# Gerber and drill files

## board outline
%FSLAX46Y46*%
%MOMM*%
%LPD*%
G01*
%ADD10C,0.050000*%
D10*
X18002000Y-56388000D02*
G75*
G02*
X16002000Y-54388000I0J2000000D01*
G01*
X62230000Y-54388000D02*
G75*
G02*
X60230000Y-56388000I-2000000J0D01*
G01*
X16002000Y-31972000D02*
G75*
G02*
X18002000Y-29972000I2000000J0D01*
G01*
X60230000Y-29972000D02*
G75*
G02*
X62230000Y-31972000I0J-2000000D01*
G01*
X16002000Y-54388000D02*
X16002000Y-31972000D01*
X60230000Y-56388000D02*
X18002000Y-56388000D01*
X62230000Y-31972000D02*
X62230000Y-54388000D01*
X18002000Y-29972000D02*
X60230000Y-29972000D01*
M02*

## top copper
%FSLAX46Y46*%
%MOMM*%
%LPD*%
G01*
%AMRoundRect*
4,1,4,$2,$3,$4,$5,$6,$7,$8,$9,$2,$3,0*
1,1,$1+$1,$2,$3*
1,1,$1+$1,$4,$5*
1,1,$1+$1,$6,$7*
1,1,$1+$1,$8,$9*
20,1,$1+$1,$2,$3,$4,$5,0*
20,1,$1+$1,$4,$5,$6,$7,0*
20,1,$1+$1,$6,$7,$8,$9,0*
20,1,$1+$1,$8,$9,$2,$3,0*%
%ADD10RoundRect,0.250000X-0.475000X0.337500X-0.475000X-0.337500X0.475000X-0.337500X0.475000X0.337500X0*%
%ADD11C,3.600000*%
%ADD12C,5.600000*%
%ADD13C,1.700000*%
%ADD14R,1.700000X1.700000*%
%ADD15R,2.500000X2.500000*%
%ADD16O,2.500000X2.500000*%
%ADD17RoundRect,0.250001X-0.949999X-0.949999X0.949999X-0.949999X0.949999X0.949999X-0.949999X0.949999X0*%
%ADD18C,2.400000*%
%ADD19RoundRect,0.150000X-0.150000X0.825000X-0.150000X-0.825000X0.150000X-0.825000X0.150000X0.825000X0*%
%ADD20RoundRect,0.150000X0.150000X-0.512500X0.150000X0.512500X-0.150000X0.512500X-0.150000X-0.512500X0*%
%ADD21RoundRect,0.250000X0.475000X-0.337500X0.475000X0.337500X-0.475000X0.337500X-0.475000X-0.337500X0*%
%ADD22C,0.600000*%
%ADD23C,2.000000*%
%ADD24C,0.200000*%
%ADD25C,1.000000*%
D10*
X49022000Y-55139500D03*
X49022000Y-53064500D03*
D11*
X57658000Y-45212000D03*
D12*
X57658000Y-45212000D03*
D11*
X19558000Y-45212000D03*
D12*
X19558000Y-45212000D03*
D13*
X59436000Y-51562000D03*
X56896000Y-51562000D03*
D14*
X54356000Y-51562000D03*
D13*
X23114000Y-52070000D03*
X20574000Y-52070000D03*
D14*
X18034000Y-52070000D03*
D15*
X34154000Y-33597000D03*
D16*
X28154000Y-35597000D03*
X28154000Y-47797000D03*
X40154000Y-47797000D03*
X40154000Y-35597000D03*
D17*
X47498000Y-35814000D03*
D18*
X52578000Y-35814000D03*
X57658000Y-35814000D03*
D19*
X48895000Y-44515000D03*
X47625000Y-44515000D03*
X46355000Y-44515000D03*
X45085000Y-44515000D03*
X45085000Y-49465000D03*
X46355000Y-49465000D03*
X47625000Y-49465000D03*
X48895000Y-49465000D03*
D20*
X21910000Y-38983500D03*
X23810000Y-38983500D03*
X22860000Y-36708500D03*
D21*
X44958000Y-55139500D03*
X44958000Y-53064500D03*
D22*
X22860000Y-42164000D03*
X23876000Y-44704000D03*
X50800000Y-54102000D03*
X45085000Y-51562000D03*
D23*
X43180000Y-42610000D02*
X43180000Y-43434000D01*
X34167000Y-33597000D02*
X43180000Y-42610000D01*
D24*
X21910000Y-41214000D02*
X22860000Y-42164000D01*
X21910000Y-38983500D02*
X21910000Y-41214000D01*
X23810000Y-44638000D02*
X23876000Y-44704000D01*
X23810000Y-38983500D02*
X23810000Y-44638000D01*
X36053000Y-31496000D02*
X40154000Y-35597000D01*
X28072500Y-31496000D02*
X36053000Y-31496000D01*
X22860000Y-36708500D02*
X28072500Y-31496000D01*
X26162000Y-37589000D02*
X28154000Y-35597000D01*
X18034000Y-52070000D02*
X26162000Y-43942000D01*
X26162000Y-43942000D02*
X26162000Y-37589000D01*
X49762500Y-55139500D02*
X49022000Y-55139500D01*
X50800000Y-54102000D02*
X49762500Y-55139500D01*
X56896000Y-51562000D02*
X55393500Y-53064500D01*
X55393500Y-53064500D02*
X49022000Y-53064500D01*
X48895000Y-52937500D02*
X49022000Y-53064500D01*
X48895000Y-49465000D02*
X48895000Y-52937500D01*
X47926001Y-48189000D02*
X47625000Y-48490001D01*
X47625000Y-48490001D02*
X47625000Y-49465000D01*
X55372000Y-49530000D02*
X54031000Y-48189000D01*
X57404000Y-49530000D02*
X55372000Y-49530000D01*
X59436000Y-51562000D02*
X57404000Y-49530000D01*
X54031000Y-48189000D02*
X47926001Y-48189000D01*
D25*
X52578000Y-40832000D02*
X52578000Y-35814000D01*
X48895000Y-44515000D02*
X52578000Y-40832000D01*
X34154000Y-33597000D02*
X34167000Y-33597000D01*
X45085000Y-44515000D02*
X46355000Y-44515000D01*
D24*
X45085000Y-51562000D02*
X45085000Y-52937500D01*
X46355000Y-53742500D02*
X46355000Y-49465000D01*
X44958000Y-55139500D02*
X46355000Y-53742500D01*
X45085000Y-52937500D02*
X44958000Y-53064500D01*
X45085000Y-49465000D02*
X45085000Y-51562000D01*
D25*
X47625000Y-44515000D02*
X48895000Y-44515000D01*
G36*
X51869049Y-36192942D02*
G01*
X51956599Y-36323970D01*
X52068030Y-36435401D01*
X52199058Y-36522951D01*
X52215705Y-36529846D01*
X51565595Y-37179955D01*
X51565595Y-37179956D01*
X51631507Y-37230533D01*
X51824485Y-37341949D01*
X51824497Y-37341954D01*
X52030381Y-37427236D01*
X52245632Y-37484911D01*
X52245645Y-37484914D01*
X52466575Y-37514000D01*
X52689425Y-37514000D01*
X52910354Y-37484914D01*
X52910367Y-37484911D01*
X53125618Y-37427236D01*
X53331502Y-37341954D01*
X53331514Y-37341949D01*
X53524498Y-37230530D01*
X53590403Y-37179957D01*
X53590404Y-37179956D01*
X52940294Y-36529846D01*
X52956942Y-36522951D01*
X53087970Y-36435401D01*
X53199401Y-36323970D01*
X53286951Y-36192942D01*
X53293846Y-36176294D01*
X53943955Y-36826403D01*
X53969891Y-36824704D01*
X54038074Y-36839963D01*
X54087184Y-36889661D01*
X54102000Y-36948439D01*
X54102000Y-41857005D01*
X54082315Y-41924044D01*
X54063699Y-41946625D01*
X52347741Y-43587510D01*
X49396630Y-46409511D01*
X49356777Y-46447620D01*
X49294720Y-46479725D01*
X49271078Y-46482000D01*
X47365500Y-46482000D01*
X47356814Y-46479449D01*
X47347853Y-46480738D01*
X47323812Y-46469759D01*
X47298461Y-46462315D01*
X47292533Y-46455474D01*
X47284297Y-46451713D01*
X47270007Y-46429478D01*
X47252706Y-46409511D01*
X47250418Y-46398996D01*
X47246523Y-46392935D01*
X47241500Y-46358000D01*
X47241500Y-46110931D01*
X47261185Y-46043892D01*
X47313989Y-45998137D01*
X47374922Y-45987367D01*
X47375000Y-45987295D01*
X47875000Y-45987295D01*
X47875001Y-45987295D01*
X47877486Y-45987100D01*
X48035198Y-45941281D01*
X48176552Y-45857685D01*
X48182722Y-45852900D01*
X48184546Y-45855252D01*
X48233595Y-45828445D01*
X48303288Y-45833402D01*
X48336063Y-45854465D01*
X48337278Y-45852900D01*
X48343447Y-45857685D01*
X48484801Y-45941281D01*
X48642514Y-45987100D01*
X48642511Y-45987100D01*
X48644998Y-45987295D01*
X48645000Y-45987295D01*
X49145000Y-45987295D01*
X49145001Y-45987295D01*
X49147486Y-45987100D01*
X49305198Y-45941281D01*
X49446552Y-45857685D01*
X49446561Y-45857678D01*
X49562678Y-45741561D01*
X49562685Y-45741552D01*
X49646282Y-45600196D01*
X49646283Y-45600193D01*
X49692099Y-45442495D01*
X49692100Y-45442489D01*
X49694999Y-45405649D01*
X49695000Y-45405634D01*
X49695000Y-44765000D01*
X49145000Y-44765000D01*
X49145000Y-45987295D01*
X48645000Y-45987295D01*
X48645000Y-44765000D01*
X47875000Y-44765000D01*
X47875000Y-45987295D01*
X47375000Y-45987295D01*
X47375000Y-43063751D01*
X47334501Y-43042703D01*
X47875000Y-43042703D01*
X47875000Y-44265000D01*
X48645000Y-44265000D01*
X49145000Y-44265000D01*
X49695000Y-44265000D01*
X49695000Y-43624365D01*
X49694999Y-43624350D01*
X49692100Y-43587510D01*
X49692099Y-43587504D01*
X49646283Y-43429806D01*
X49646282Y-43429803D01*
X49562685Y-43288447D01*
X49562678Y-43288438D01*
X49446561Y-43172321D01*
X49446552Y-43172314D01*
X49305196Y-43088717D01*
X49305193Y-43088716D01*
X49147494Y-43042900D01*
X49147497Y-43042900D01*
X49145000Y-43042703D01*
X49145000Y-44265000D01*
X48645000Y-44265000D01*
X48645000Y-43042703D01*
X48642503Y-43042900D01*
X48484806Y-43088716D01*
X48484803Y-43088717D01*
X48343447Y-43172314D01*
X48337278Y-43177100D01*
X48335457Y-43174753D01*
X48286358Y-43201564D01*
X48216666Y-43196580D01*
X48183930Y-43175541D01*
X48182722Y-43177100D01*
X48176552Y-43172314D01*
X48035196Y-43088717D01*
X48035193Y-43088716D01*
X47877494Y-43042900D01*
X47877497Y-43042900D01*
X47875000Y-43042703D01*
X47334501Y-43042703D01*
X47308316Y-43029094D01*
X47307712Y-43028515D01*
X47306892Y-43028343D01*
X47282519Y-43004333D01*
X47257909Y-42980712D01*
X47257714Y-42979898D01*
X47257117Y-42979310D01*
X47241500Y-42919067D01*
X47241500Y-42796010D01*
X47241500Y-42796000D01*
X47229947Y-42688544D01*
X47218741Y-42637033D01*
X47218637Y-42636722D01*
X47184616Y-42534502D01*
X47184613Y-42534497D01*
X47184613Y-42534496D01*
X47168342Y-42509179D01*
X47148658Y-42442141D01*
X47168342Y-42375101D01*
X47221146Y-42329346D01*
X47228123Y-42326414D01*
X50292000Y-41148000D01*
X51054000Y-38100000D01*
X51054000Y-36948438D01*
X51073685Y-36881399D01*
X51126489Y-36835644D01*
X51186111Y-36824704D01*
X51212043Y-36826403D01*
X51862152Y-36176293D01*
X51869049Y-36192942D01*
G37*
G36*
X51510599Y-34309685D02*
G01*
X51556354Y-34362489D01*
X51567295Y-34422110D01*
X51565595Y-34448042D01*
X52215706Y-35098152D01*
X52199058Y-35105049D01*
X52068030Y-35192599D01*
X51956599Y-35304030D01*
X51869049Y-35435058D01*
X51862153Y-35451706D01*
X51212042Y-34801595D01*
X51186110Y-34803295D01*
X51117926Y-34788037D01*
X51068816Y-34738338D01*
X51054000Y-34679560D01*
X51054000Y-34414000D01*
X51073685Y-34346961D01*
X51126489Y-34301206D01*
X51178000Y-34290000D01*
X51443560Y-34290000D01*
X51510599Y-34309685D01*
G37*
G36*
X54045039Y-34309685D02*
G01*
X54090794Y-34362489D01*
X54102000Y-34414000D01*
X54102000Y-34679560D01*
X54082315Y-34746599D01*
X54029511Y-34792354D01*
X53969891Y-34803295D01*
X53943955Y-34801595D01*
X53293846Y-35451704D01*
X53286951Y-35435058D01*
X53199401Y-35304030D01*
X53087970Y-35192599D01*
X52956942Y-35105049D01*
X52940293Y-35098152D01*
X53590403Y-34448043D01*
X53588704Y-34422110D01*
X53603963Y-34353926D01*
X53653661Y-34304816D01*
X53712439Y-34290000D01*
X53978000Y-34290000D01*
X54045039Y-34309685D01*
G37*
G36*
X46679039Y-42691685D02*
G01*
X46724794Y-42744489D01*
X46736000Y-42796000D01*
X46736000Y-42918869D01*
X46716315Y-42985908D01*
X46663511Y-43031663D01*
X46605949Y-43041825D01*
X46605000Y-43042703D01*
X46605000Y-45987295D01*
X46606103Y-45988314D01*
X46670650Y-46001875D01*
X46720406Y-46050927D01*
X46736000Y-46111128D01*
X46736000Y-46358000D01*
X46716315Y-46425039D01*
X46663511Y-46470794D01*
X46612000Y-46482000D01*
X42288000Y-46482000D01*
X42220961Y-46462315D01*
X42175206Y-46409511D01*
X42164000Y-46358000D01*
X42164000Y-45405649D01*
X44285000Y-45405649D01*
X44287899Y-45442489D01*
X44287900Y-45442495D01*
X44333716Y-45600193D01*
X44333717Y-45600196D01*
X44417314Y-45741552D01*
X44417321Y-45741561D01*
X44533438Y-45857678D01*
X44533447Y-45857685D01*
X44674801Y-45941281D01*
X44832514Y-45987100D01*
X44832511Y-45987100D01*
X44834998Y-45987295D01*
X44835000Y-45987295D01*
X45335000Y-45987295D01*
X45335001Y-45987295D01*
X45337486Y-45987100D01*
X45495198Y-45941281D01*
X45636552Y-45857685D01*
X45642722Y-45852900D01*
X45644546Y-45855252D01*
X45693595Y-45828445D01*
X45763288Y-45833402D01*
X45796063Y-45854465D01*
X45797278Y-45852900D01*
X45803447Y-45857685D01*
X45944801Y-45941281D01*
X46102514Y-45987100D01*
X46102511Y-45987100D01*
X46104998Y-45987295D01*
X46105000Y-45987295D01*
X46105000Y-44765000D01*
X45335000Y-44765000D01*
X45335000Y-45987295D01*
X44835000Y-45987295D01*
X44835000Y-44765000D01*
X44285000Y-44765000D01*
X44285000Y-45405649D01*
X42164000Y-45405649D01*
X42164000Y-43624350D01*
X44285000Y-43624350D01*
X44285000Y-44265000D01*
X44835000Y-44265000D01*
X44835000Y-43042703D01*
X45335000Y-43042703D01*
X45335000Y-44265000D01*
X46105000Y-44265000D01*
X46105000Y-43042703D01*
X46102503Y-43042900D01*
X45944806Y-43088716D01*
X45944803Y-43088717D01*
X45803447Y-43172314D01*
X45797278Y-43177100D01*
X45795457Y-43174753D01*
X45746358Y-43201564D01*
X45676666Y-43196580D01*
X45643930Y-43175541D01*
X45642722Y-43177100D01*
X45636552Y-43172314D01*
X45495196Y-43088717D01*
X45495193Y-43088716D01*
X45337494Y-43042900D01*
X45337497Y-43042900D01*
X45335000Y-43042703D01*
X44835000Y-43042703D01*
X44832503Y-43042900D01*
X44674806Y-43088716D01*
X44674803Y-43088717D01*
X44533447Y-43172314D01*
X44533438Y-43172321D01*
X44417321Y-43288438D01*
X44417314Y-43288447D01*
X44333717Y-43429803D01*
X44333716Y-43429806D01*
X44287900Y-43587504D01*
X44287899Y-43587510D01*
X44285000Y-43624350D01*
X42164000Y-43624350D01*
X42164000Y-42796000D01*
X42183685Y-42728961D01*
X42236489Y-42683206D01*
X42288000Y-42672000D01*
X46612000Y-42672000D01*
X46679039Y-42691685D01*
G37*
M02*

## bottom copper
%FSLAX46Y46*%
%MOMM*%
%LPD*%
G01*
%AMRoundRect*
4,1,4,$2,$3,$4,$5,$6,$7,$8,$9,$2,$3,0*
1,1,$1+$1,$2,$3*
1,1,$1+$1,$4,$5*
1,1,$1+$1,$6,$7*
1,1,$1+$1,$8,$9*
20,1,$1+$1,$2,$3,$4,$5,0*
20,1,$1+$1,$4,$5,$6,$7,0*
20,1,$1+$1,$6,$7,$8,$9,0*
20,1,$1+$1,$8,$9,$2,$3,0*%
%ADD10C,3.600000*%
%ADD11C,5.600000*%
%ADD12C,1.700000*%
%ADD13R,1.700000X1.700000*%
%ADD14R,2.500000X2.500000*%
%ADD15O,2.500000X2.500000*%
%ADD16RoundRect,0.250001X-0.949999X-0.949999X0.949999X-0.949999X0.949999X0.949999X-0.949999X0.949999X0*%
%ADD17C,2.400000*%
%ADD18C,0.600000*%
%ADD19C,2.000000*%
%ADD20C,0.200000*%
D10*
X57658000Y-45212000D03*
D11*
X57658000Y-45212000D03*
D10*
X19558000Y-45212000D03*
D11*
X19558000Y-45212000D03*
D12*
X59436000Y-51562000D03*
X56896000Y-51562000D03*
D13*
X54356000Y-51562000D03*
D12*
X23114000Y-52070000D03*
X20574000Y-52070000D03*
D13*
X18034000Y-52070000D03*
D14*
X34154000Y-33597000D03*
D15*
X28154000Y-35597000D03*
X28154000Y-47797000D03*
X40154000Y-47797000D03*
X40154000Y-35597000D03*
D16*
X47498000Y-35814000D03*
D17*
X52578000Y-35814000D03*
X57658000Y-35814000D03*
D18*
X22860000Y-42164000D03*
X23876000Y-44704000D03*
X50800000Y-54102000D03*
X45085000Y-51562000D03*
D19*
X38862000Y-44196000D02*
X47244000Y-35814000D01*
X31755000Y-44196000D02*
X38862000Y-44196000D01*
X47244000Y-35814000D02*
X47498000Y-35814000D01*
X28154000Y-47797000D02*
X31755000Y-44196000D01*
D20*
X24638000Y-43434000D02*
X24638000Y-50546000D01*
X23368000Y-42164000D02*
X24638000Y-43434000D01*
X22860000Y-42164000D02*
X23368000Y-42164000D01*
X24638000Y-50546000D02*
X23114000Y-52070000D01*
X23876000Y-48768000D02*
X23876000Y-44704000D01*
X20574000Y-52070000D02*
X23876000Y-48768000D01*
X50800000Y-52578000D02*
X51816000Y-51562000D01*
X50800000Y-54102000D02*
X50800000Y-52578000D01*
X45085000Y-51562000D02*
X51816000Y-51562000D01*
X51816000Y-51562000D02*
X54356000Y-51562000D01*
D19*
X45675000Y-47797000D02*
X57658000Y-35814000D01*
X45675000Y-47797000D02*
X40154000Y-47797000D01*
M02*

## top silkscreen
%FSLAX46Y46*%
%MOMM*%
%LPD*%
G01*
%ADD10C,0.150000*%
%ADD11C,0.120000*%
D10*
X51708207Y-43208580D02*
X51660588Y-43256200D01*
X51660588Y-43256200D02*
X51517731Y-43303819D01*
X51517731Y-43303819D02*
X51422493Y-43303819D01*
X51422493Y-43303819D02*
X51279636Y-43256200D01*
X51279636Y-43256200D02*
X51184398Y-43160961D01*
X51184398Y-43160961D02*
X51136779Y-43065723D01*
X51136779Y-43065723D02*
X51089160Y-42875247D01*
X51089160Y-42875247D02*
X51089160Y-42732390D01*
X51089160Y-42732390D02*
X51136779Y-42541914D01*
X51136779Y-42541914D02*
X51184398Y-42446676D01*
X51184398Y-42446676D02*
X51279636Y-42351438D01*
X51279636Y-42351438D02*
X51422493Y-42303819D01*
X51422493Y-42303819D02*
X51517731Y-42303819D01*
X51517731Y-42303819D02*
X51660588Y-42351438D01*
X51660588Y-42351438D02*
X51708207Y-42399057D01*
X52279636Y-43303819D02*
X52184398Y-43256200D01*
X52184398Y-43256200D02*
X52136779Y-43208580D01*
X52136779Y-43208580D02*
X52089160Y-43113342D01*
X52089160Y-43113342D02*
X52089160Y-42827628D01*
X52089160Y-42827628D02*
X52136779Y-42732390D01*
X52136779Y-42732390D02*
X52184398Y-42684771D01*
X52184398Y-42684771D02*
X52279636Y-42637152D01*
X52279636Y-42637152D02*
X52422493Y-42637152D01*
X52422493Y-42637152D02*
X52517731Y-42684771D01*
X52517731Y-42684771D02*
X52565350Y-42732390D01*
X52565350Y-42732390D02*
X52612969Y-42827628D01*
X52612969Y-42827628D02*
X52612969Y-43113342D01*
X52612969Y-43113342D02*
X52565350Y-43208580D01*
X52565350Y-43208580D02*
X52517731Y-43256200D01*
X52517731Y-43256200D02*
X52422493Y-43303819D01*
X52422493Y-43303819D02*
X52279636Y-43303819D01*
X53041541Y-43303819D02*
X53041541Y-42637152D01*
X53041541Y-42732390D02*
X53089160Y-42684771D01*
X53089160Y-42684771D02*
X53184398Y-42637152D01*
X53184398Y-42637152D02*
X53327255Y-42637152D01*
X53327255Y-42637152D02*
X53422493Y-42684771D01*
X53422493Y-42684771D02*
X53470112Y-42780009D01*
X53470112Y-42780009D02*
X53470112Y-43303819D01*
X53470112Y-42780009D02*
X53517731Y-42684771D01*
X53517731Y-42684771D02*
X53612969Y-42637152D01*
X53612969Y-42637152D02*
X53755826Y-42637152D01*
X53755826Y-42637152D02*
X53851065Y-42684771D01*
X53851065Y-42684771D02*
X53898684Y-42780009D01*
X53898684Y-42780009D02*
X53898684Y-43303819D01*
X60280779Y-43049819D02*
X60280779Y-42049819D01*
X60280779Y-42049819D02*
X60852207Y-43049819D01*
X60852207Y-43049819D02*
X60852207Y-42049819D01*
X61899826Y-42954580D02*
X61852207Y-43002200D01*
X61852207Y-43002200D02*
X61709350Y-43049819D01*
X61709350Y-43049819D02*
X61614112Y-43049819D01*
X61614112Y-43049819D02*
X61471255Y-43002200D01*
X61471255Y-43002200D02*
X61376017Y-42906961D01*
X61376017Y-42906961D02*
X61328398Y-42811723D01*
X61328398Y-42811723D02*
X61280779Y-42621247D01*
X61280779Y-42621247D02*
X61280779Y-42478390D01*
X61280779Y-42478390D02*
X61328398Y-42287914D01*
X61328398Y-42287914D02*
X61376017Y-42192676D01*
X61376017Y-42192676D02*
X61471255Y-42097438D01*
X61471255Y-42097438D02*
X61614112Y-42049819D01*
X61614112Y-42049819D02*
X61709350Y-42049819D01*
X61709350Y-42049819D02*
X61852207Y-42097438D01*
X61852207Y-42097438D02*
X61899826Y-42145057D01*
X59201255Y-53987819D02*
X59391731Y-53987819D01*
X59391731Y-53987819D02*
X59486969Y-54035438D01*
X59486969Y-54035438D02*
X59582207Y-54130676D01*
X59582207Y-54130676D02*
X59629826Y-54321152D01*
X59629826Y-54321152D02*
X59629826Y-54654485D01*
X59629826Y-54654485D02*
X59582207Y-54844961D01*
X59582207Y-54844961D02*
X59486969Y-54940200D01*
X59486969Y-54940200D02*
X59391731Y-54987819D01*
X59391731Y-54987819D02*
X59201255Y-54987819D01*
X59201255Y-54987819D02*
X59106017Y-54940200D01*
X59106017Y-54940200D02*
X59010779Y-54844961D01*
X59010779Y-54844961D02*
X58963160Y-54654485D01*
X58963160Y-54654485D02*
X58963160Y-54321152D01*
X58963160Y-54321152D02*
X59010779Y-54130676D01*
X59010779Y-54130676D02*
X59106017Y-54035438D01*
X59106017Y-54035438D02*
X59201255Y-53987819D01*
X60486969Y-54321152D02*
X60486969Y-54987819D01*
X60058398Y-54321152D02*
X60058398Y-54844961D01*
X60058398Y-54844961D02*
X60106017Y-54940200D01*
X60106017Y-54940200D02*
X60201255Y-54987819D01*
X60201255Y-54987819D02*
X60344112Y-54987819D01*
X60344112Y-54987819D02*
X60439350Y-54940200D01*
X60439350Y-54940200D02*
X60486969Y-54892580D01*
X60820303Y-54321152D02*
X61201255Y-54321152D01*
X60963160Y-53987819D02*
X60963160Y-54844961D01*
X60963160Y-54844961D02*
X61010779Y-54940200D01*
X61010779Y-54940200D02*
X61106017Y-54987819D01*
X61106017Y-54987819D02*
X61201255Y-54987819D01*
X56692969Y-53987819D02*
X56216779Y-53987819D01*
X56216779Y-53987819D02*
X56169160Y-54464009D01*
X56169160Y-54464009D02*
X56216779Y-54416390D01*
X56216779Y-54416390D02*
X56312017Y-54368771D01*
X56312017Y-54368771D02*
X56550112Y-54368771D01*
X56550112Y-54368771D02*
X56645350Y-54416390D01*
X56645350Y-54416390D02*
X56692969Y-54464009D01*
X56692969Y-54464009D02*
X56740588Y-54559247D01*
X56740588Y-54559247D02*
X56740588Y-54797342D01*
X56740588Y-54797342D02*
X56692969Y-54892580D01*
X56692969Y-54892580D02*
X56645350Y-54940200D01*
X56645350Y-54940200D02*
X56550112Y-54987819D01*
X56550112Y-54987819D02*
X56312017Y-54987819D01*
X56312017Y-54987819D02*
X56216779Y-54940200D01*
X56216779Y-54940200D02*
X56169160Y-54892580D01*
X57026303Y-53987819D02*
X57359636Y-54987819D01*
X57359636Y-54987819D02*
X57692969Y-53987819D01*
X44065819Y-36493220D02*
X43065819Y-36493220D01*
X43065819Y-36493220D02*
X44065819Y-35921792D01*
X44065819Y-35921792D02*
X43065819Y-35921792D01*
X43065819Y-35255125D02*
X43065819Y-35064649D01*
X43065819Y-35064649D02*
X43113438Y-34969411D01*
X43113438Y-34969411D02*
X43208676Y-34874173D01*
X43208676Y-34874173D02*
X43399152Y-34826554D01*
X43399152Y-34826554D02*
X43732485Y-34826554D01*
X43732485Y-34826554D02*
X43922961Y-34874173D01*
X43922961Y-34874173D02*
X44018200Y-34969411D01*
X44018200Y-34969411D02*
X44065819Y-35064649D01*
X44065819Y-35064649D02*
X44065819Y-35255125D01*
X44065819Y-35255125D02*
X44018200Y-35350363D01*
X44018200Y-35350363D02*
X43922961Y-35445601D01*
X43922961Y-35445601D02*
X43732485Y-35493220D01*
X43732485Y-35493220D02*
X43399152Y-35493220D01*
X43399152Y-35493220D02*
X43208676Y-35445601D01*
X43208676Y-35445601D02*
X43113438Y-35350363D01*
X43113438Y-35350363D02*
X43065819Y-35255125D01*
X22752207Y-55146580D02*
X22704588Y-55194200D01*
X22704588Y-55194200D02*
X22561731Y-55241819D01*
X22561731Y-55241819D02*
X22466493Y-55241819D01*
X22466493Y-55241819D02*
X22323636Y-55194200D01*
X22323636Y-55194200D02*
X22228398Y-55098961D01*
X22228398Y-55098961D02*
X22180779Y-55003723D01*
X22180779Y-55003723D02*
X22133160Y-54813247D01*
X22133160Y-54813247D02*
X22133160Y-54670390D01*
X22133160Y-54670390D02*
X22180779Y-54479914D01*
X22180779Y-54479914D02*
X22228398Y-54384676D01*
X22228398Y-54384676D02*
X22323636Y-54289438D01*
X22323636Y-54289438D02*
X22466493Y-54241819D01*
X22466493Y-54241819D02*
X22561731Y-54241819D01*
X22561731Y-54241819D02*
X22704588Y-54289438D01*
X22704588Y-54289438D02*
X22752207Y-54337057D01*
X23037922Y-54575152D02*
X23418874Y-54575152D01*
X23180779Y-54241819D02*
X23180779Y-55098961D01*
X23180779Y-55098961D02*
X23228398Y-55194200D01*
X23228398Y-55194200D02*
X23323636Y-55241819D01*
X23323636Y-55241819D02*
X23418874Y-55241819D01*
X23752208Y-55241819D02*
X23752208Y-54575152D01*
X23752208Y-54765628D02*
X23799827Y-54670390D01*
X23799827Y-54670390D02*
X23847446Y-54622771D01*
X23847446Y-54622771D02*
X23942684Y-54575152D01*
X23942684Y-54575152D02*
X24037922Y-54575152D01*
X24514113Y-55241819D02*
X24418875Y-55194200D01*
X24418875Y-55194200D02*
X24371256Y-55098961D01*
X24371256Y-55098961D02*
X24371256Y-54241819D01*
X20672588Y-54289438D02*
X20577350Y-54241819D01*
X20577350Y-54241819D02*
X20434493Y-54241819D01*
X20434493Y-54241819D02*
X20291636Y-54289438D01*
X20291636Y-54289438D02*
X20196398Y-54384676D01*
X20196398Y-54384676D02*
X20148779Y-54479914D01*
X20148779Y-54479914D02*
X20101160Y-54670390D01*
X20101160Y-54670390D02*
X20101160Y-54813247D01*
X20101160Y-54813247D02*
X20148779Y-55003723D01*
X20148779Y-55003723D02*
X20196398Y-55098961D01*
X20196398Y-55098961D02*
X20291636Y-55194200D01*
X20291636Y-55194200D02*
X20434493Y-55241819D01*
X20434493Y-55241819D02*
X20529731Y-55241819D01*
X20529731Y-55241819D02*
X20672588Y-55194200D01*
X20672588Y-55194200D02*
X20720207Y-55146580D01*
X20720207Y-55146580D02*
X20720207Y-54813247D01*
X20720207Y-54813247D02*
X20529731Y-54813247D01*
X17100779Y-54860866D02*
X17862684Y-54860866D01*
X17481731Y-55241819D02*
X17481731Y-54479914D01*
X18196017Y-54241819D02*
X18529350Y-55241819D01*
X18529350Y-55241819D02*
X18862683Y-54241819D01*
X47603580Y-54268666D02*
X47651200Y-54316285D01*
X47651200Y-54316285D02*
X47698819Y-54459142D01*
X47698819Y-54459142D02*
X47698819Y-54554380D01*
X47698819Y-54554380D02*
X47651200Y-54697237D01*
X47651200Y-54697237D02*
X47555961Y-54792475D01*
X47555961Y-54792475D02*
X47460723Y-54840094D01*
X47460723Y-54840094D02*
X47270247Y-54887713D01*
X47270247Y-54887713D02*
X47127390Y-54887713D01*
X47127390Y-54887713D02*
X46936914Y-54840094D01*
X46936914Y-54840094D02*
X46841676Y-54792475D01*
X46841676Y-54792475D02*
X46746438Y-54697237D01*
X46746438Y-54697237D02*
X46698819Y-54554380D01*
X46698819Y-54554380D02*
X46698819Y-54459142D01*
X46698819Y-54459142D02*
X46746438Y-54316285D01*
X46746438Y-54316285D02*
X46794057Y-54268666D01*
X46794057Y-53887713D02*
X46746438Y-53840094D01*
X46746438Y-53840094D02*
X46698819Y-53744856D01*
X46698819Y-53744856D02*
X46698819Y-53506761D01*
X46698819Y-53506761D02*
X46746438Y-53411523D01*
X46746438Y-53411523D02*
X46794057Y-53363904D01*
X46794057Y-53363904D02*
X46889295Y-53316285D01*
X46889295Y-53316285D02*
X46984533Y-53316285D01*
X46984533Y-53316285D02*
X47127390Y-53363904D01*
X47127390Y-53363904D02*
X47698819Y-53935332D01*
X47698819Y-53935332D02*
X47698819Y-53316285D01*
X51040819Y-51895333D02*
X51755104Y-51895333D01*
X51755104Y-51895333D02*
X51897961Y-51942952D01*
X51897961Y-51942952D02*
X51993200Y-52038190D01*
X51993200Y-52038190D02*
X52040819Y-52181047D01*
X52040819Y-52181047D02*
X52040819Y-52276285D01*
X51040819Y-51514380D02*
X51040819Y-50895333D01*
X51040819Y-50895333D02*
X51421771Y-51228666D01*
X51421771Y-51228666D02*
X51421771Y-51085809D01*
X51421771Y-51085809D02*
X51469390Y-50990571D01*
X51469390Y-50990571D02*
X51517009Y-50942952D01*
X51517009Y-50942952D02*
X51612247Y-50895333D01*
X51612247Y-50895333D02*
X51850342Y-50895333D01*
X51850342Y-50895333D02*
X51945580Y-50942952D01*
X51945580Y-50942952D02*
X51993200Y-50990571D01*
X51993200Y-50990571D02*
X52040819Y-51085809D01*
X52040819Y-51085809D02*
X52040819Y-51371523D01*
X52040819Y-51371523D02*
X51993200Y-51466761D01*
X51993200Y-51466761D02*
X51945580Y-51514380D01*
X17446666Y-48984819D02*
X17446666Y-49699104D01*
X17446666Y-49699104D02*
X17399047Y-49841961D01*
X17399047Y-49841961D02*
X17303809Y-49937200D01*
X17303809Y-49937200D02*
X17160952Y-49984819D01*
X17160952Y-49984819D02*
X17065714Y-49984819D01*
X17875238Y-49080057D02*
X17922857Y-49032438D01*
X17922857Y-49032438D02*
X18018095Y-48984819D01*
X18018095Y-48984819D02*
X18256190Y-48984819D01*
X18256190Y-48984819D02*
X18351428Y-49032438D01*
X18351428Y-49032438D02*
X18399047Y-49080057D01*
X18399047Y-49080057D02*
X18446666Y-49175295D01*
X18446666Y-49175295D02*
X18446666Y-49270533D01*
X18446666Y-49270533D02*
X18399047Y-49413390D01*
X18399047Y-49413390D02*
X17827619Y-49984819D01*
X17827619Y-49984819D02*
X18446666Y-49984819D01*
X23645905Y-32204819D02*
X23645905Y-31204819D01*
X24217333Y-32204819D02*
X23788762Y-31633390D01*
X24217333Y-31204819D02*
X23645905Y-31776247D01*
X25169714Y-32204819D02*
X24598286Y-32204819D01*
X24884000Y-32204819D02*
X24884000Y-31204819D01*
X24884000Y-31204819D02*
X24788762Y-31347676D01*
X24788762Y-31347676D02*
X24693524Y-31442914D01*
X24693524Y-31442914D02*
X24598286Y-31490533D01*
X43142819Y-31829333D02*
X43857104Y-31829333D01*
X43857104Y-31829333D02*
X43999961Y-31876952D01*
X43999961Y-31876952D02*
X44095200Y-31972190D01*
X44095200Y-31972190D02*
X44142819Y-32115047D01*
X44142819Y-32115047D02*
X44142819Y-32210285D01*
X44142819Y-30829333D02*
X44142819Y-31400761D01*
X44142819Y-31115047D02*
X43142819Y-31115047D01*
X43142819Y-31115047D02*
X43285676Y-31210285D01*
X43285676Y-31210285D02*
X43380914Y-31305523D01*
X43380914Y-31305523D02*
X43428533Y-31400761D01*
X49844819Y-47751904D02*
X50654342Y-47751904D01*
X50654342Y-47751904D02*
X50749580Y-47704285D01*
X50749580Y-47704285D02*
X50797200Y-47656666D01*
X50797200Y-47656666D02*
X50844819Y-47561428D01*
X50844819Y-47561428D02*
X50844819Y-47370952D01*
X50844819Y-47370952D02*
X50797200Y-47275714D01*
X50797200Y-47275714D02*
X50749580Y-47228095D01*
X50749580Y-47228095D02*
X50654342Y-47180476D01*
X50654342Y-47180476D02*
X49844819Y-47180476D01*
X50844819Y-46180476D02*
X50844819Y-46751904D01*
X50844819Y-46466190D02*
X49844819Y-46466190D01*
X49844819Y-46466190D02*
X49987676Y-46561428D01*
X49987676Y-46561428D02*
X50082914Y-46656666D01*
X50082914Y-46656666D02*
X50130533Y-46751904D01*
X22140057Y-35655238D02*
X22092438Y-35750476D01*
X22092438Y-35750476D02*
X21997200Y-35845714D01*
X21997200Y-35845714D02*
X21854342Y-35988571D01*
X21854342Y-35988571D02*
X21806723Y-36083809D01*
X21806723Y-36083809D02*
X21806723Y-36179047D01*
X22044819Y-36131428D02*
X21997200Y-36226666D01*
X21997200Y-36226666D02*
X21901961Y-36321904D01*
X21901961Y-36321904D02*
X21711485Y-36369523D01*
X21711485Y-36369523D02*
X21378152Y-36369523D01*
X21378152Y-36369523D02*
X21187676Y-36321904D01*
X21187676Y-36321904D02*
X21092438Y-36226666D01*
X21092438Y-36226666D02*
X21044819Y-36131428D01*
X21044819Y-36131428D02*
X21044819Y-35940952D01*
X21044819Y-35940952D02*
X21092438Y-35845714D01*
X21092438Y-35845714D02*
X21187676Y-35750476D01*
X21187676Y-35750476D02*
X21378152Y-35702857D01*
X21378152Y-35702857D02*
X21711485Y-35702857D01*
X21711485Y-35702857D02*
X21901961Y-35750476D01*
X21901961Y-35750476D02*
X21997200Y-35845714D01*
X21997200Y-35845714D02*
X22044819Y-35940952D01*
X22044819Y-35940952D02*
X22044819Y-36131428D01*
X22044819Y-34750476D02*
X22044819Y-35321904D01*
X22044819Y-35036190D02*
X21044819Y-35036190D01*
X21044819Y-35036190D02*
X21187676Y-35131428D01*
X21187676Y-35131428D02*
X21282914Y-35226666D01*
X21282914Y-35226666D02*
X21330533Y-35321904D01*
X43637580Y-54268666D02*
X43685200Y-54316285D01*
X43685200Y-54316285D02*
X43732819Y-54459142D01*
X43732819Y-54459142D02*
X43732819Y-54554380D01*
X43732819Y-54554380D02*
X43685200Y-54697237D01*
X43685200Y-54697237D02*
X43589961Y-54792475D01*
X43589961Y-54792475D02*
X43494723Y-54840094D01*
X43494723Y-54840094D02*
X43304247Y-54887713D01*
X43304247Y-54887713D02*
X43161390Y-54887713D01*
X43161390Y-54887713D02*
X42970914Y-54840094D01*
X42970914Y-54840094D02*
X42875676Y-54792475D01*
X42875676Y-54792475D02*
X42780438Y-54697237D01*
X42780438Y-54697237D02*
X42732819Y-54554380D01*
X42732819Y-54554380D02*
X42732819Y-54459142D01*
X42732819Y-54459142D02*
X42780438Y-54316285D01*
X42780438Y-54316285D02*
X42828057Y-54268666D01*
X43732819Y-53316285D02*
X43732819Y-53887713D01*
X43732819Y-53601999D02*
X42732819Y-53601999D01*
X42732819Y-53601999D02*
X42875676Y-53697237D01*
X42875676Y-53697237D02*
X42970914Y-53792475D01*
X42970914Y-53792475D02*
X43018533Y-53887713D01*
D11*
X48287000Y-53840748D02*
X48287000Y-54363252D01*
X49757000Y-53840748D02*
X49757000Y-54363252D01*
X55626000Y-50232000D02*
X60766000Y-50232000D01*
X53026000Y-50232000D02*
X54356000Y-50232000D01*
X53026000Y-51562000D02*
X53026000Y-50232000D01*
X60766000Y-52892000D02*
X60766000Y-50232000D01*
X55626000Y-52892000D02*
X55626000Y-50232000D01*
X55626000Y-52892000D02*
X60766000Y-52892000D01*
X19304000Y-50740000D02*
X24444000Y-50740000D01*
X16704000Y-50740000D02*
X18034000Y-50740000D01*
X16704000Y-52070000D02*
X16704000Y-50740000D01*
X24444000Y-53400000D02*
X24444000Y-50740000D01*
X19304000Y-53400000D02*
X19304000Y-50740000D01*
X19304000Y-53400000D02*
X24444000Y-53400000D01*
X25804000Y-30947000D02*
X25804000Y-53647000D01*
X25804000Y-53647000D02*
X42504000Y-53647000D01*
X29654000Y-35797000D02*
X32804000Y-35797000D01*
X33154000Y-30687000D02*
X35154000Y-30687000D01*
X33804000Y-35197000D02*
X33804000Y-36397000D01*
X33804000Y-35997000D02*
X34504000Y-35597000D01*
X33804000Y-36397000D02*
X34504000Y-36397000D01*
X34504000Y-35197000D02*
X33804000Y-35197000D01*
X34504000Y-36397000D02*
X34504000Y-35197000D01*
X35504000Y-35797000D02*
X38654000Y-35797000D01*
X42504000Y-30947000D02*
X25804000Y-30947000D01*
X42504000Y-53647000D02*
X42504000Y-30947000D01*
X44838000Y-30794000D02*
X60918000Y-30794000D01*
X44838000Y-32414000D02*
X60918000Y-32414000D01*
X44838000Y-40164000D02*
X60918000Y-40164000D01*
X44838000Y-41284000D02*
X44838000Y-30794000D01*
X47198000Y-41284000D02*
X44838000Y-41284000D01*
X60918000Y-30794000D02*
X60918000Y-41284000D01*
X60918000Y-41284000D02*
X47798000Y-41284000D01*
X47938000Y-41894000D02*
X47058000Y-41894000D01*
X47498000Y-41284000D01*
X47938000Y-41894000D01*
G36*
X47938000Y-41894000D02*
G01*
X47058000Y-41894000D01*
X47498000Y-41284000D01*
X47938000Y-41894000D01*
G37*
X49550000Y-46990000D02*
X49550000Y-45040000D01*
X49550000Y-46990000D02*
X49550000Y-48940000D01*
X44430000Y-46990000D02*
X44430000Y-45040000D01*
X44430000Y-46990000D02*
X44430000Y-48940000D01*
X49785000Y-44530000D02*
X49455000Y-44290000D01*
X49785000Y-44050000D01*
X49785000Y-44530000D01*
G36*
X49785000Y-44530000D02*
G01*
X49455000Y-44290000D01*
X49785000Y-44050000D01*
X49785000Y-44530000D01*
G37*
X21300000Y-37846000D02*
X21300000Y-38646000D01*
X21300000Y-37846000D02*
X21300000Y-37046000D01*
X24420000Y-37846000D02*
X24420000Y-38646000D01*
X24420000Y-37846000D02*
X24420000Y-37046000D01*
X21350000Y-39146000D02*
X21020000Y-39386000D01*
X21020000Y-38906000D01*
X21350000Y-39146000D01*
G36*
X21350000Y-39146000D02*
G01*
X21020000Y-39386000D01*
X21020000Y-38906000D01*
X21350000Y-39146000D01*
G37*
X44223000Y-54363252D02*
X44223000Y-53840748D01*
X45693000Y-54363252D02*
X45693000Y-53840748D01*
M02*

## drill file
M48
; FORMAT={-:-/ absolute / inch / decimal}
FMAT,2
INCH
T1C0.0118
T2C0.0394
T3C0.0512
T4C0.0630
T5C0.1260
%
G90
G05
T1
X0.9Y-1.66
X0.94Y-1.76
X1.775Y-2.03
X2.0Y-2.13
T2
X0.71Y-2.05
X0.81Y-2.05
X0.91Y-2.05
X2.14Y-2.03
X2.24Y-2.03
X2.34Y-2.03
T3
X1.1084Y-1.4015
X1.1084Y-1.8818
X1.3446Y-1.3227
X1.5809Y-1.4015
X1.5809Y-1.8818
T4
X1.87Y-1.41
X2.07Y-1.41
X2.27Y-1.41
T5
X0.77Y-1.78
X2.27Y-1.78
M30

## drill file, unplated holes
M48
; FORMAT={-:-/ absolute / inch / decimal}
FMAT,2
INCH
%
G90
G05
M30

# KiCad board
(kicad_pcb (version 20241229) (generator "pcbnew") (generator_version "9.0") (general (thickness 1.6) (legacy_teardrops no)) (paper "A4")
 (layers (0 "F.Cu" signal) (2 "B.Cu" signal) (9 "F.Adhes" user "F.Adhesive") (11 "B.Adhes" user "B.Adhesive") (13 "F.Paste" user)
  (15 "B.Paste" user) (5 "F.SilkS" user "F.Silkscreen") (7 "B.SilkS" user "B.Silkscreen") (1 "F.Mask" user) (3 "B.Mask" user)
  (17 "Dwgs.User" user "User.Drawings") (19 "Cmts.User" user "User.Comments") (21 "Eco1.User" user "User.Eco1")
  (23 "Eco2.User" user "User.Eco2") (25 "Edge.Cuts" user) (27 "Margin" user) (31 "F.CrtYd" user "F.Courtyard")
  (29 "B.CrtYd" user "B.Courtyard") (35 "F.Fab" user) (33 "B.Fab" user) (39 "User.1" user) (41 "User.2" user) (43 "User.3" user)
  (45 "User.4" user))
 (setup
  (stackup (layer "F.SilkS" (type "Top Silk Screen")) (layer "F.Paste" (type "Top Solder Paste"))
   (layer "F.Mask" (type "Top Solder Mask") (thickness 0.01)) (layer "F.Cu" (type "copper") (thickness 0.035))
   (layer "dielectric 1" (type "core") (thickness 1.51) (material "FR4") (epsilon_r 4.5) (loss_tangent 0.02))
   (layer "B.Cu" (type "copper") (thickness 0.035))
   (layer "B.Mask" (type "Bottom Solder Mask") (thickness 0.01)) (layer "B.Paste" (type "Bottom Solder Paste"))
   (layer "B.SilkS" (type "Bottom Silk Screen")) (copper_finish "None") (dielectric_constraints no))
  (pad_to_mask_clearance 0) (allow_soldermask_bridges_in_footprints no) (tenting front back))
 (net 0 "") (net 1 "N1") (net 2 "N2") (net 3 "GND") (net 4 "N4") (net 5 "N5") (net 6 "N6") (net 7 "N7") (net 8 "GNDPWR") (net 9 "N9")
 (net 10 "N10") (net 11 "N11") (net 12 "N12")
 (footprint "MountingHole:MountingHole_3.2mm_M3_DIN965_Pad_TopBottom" (layer "F.Cu") (at 19.558 45.212)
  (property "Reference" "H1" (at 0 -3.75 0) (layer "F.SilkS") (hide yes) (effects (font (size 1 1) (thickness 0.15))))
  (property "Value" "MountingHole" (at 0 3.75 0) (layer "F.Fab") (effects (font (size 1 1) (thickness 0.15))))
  (pad "1" thru_hole circle (at 0 0) (size 3.6 3.6) (drill 3.2) (layers "*.Cu" "*.Mask") (remove_unused_layers no) (zone_connect 2))
  (pad "1" connect circle (at 0 0) (size 5.6 5.6) (layers "F.Cu" "F.Mask") (zone_connect 2))
  (pad "1" connect circle (at 0 0) (size 5.6 5.6) (layers "B.Cu" "B.Mask") (zone_connect 2)))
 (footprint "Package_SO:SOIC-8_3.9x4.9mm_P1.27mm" (layer "F.Cu") (at 46.99 46.99 -90)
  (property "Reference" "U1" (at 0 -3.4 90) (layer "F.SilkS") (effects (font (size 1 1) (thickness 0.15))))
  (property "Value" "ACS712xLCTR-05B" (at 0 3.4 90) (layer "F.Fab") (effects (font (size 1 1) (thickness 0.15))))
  (fp_line (start 0 2.56) (end -1.95 2.56) (stroke (width 0.12) (type solid)) (layer "F.SilkS"))
  (fp_line (start 0 2.56) (end 1.95 2.56) (stroke (width 0.12) (type solid)) (layer "F.SilkS"))
  (fp_line (start 0 -2.56) (end -1.95 -2.56) (stroke (width 0.12) (type solid)) (layer "F.SilkS"))
  (fp_line (start 0 -2.56) (end 1.95 -2.56) (stroke (width 0.12) (type solid)) (layer "F.SilkS"))
  (fp_poly (pts (xy -2.7 -2.465) (xy -2.94 -2.795) (xy -2.46 -2.795)) (stroke (width 0.12) (type solid)) (fill yes) (layer "F.SilkS"))
  (pad "1" smd roundrect (at -2.475 -1.905 270) (size 1.95 0.6) (layers "F.Cu" "F.Mask" "F.Paste") (roundrect_rratio 0.25) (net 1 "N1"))
  (pad "2" smd roundrect (at -2.475 -0.635 270) (size 1.95 0.6) (layers "F.Cu" "F.Mask" "F.Paste") (roundrect_rratio 0.25) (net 1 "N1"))
  (pad "3" smd roundrect (at -2.475 0.635 270) (size 1.95 0.6) (layers "F.Cu" "F.Mask" "F.Paste") (roundrect_rratio 0.25) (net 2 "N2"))
  (pad "4" smd roundrect (at -2.475 1.905 270) (size 1.95 0.6) (layers "F.Cu" "F.Mask" "F.Paste") (roundrect_rratio 0.25) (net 2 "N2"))
  (pad "5" smd roundrect (at 2.475 1.905 270) (size 1.95 0.6) (layers "F.Cu" "F.Mask" "F.Paste") (roundrect_rratio 0.25) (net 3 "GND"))
  (pad "6" smd roundrect (at 2.475 0.635 270) (size 1.95 0.6) (layers "F.Cu" "F.Mask" "F.Paste") (roundrect_rratio 0.25) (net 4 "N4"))
  (pad "7" smd roundrect (at 2.475 -0.635 270) (size 1.95 0.6) (layers "F.Cu" "F.Mask" "F.Paste") (roundrect_rratio 0.25) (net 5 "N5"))
  (pad "8" smd roundrect (at 2.475 -1.905 270) (size 1.95 0.6) (layers "F.Cu" "F.Mask" "F.Paste") (roundrect_rratio 0.25) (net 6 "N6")))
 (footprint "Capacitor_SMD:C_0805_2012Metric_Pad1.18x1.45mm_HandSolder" (layer "F.Cu") (at 44.958 54.102 90)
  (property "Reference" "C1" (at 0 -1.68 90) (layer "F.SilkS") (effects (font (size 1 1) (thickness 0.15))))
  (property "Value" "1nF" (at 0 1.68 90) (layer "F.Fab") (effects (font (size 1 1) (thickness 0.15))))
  (fp_line (start -0.261252 -0.735) (end 0.261252 -0.735) (stroke (width 0.12) (type solid)) (layer "F.SilkS"))
  (fp_line (start -0.261252 0.735) (end 0.261252 0.735) (stroke (width 0.12) (type solid)) (layer "F.SilkS"))
  (pad "1" smd roundrect (at -1.0375 0 90) (size 1.175 1.45) (layers "F.Cu" "F.Mask" "F.Paste") (roundrect_rratio 0.212766) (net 4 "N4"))
  (pad "2" smd roundrect (at 1.0375 0 90) (size 1.175 1.45) (layers "F.Cu" "F.Mask" "F.Paste") (roundrect_rratio 0.212766) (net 3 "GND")))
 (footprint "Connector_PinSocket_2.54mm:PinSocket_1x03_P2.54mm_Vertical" (layer "F.Cu") (at 18.034 52.07 90)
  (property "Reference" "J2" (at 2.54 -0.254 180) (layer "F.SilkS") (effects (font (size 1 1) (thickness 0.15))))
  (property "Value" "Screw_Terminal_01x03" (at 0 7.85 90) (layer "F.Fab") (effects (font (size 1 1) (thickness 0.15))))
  (fp_line (start 1.33 -1.33) (end 1.33 0) (stroke (width 0.12) (type solid)) (layer "F.SilkS"))
  (fp_line (start 0 -1.33) (end 1.33 -1.33) (stroke (width 0.12) (type solid)) (layer "F.SilkS"))
  (fp_line (start 1.33 1.27) (end 1.33 6.41) (stroke (width 0.12) (type solid)) (layer "F.SilkS"))
  (fp_line (start -1.33 1.27) (end 1.33 1.27) (stroke (width 0.12) (type solid)) (layer "F.SilkS"))
  (fp_line (start -1.33 1.27) (end -1.33 6.41) (stroke (width 0.12) (type solid)) (layer "F.SilkS"))
  (fp_line (start -1.33 6.41) (end 1.33 6.41) (stroke (width 0.12) (type solid)) (layer "F.SilkS"))
  (pad "1" thru_hole rect (at 0 0 90) (size 1.7 1.7) (drill 1) (layers "*.Cu" "*.Mask") (remove_unused_layers no) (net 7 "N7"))
  (pad "2" thru_hole circle (at 0 2.54 90) (size 1.7 1.7) (drill 1) (layers "*.Cu" "*.Mask") (remove_unused_layers no) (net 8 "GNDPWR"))
  (pad "3" thru_hole circle (at 0 5.08 90) (size 1.7 1.7) (drill 1) (layers "*.Cu" "*.Mask") (remove_unused_layers no) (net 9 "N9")))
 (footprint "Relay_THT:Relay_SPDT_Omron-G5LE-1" (layer "F.Cu") (at 34.154 33.597)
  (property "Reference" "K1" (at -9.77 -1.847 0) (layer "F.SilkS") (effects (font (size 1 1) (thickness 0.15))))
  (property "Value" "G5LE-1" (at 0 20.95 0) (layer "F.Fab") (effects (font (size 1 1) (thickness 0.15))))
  (fp_line (start -8.35 -2.65) (end -8.35 20.05) (stroke (width 0.12) (type solid)) (layer "F.SilkS"))
  (fp_line (start -8.35 20.05) (end 8.35 20.05) (stroke (width 0.12) (type solid)) (layer "F.SilkS"))
  (fp_line (start -4.5 2.2) (end -1.35 2.2) (stroke (width 0.12) (type solid)) (layer "F.SilkS"))
  (fp_line (start -1 -2.91) (end 1 -2.91) (stroke (width 0.12) (type solid)) (layer "F.SilkS"))
  (fp_line (start -0.35 1.6) (end -0.35 2.8) (stroke (width 0.12) (type solid)) (layer "F.SilkS"))
  (fp_line (start -0.35 2.4) (end 0.35 2) (stroke (width 0.12) (type solid)) (layer "F.SilkS"))
  (fp_line (start -0.35 2.8) (end 0.35 2.8) (stroke (width 0.12) (type solid)) (layer "F.SilkS"))
  (fp_line (start 0.35 1.6) (end -0.35 1.6) (stroke (width 0.12) (type solid)) (layer "F.SilkS"))
  (fp_line (start 0.35 2.8) (end 0.35 1.6) (stroke (width 0.12) (type solid)) (layer "F.SilkS"))
  (fp_line (start 1.35 2.2) (end 4.5 2.2) (stroke (width 0.12) (type solid)) (layer "F.SilkS"))
  (fp_line (start 8.35 -2.65) (end -8.35 -2.65) (stroke (width 0.12) (type solid)) (layer "F.SilkS"))
  (fp_line (start 8.35 20.05) (end 8.35 -2.65) (stroke (width 0.12) (type solid)) (layer "F.SilkS"))
  (pad "1" thru_hole rect (at 0 0) (size 2.5 2.5) (drill 1.3) (layers "*.Cu" "*.Mask") (remove_unused_layers no) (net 2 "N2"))
  (pad "2" thru_hole oval (at -6 2) (size 2.5 2.5) (drill 1.3) (layers "*.Cu" "*.Mask") (remove_unused_layers no) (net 7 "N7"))
  (pad "3" thru_hole oval (at -6 14.2) (size 2.5 2.5) (drill 1.3) (layers "*.Cu" "*.Mask") (remove_unused_layers no) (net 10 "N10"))
  (pad "4" thru_hole oval (at 6 14.2) (size 2.5 2.5) (drill 1.3) (layers "*.Cu" "*.Mask") (remove_unused_layers no) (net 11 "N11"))
  (pad "5" thru_hole oval (at 6 2) (size 2.5 2.5) (drill 1.3) (layers "*.Cu" "*.Mask") (remove_unused_layers no) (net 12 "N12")))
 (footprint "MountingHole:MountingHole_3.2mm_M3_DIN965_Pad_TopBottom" (layer "F.Cu") (at 57.658 45.212)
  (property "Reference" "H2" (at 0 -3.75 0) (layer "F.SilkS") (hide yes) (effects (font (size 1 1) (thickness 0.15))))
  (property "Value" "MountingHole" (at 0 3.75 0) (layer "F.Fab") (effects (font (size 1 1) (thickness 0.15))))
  (pad "1" thru_hole circle (at 0 0) (size 3.6 3.6) (drill 3.2) (layers "*.Cu" "*.Mask") (remove_unused_layers no) (zone_connect 2))
  (pad "1" connect circle (at 0 0) (size 5.6 5.6) (layers "F.Cu" "F.Mask") (zone_connect 2))
  (pad "1" connect circle (at 0 0) (size 5.6 5.6) (layers "B.Cu" "B.Mask") (zone_connect 2)))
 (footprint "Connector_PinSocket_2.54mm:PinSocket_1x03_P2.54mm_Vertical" (layer "F.Cu") (at 54.356 51.562 90)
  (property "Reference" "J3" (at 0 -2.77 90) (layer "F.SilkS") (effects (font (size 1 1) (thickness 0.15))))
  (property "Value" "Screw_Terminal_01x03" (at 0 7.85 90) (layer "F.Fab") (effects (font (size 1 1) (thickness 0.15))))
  (fp_line (start 1.33 -1.33) (end 1.33 0) (stroke (width 0.12) (type solid)) (layer "F.SilkS"))
  (fp_line (start 0 -1.33) (end 1.33 -1.33) (stroke (width 0.12) (type solid)) (layer "F.SilkS"))
  (fp_line (start 1.33 1.27) (end 1.33 6.41) (stroke (width 0.12) (type solid)) (layer "F.SilkS"))
  (fp_line (start -1.33 1.27) (end 1.33 1.27) (stroke (width 0.12) (type solid)) (layer "F.SilkS"))
  (fp_line (start -1.33 1.27) (end -1.33 6.41) (stroke (width 0.12) (type solid)) (layer "F.SilkS"))
  (fp_line (start -1.33 6.41) (end 1.33 6.41) (stroke (width 0.12) (type solid)) (layer "F.SilkS"))
  (pad "1" thru_hole rect (at 0 0 90) (size 1.7 1.7) (drill 1) (layers "*.Cu" "*.Mask") (remove_unused_layers no) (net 3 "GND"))
  (pad "2" thru_hole circle (at 0 2.54 90) (size 1.7 1.7) (drill 1) (layers "*.Cu" "*.Mask") (remove_unused_layers no) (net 6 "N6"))
  (pad "3" thru_hole circle (at 0 5.08 90) (size 1.7 1.7) (drill 1) (layers "*.Cu" "*.Mask") (remove_unused_layers no) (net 5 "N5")))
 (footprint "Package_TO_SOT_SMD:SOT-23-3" (layer "F.Cu") (at 22.86 37.846 90)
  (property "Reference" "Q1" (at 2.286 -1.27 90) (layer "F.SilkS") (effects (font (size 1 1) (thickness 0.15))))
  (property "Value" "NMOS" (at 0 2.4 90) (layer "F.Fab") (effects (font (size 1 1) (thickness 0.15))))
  (fp_line (start 0 -1.56) (end 0.8 -1.56) (stroke (width 0.12) (type solid)) (layer "F.SilkS"))
  (fp_line (start 0 -1.56) (end -0.8 -1.56) (stroke (width 0.12) (type solid)) (layer "F.SilkS"))
  (fp_line (start 0 1.56) (end 0.8 1.56) (stroke (width 0.12) (type solid)) (layer "F.SilkS"))
  (fp_line (start 0 1.56) (end -0.8 1.56) (stroke (width 0.12) (type solid)) (layer "F.SilkS"))
  (fp_poly (pts (xy -1.3 -1.51) (xy -1.54 -1.84) (xy -1.06 -1.84)) (stroke (width 0.12) (type solid)) (fill yes) (layer "F.SilkS"))
  (pad "1" smd roundrect (at -1.1375 -0.95 90) (size 1.325 0.6) (layers "F.Cu" "F.Mask" "F.Paste") (roundrect_rratio 0.25) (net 9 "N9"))
  (pad "2" smd roundrect (at -1.1375 0.95 90) (size 1.325 0.6) (layers "F.Cu" "F.Mask" "F.Paste") (roundrect_rratio 0.25) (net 8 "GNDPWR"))
  (pad "3" smd roundrect (at 1.1375 0 90) (size 1.325 0.6) (layers "F.Cu" "F.Mask" "F.Paste") (roundrect_rratio 0.25) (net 12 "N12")))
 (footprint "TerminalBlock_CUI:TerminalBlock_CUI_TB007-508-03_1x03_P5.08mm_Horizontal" (layer "F.Cu") (at 47.498 35.814)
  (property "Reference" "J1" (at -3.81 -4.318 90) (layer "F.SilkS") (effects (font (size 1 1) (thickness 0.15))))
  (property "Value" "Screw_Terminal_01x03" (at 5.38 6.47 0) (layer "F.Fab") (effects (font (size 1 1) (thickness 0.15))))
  (fp_line (start -2.66 -5.02) (end 13.42 -5.02) (stroke (width 0.12) (type solid)) (layer "F.SilkS"))
  (fp_line (start -2.66 -3.4) (end 13.42 -3.4) (stroke (width 0.12) (type solid)) (layer "F.SilkS"))
  (fp_line (start -2.66 4.35) (end 13.42 4.35) (stroke (width 0.12) (type solid)) (layer "F.SilkS"))
  (fp_line (start -2.66 5.47) (end -2.66 -5.02) (stroke (width 0.12) (type solid)) (layer "F.SilkS"))
  (fp_line (start -0.3 5.47) (end -2.66 5.47) (stroke (width 0.12) (type solid)) (layer "F.SilkS"))
  (fp_line (start 13.42 -5.02) (end 13.42 5.47) (stroke (width 0.12) (type solid)) (layer "F.SilkS"))
  (fp_line (start 13.42 5.47) (end 0.3 5.47) (stroke (width 0.12) (type solid)) (layer "F.SilkS"))
  (fp_poly (pts (xy 0 5.47) (xy 0.44 6.08) (xy -0.44 6.08)) (stroke (width 0.12) (type solid)) (fill yes) (layer "F.SilkS"))
  (pad "1" thru_hole roundrect (at 0 0) (size 2.4 2.4) (drill 1.6) (layers "*.Cu" "*.Mask") (remove_unused_layers no)
   (roundrect_rratio 0.104167) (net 10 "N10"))
  (pad "2" thru_hole circle (at 5.08 0) (size 2.4 2.4) (drill 1.6) (layers "*.Cu" "*.Mask") (remove_unused_layers no) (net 1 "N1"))
  (pad "3" thru_hole circle (at 10.16 0) (size 2.4 2.4) (drill 1.6) (layers "*.Cu" "*.Mask") (remove_unused_layers no) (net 11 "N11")))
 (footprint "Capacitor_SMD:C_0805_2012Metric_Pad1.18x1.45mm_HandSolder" (layer "F.Cu") (at 49.022 54.102 -90)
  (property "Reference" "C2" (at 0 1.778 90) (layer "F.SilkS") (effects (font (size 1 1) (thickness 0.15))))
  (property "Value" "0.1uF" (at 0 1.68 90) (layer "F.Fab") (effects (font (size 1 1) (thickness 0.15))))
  (fp_line (start -0.261252 0.735) (end 0.261252 0.735) (stroke (width 0.12) (type solid)) (layer "F.SilkS"))
  (fp_line (start -0.261252 -0.735) (end 0.261252 -0.735) (stroke (width 0.12) (type solid)) (layer "F.SilkS"))
  (pad "1" smd roundrect (at -1.0375 0 270) (size 1.175 1.45) (layers "F.Cu" "F.Mask" "F.Paste") (roundrect_rratio 0.212766) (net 6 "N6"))
  (pad "2" smd roundrect (at 1.0375 0 270) (size 1.175 1.45) (layers "F.Cu" "F.Mask" "F.Paste") (roundrect_rratio 0.212766) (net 3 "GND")))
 (gr_line (start 60.23 56.388) (end 18.002 56.388) (stroke (width 0.05) (type default)) (layer "Edge.Cuts"))
 (gr_line (start 62.23 31.972) (end 62.23 54.388) (stroke (width 0.05) (type default)) (layer "Edge.Cuts"))
 (gr_arc (start 18.002 56.388) (mid 16.587786 55.802214) (end 16.002 54.388) (stroke (width 0.05) (type default)) (layer "Edge.Cuts"))
 (gr_arc (start 16.002 31.972) (mid 16.587786 30.557786) (end 18.002 29.972) (stroke (width 0.05) (type default)) (layer "Edge.Cuts"))
 (gr_line (start 18.002 29.972) (end 60.23 29.972) (stroke (width 0.05) (type default)) (layer "Edge.Cuts"))
 (gr_arc (start 62.23 54.388) (mid 61.644214 55.802214) (end 60.23 56.388) (stroke (width 0.05) (type default)) (layer "Edge.Cuts"))
 (gr_line (start 16.002 54.388) (end 16.002 31.972) (stroke (width 0.05) (type default)) (layer "Edge.Cuts"))
 (gr_arc (start 60.23 29.972) (mid 61.644214 30.557786) (end 62.23 31.972) (stroke (width 0.05) (type default)) (layer "Edge.Cuts"))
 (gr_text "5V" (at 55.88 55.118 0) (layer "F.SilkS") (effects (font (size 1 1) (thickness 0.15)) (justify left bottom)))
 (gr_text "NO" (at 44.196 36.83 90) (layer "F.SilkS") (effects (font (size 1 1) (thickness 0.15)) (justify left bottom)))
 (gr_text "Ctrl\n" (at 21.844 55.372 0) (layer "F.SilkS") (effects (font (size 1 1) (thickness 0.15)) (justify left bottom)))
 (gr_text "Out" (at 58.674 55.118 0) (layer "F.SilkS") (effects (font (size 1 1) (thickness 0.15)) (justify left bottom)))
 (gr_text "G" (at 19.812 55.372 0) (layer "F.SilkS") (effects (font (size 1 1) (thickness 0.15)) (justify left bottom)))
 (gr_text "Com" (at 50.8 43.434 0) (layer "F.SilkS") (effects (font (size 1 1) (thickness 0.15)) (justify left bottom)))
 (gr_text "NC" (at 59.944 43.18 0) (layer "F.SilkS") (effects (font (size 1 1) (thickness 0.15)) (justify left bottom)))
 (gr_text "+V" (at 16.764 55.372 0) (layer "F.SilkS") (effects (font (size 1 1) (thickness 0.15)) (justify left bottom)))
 (segment (start 46.355 53.7425) (end 46.355 49.465) (width 0.2) (layer "F.Cu") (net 4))
 (segment (start 44.958 55.1395) (end 46.355 53.7425) (width 0.2) (layer "F.Cu") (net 4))
 (segment (start 45.085 51.562) (end 45.085 52.9375) (width 0.2) (layer "F.Cu") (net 3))
 (segment (start 50.8 54.102) (end 49.7625 55.1395) (width 0.2) (layer "F.Cu") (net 3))
 (segment (start 49.7625 55.1395) (end 49.022 55.1395) (width 0.2) (layer "F.Cu") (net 3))
 (segment (start 45.085 52.9375) (end 44.958 53.0645) (width 0.2) (layer "F.Cu") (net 3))
 (segment (start 45.085 49.465) (end 45.085 51.562) (width 0.2) (layer "F.Cu") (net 3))
 (via (at 50.8 54.102) (size 0.6) (drill 0.3) (layers "F.Cu" "B.Cu") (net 3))
 (via (at 45.085 51.562) (size 0.6) (drill 0.3) (layers "F.Cu" "B.Cu") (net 3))
 (segment (start 50.8 54.102) (end 50.8 52.578) (width 0.2) (layer "B.Cu") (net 3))
 (segment (start 50.8 52.578) (end 51.816 51.562) (width 0.2) (layer "B.Cu") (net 3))
 (segment (start 45.085 51.562) (end 51.816 51.562) (width 0.2) (layer "B.Cu") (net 3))
 (segment (start 51.816 51.562) (end 54.356 51.562) (width 0.2) (layer "B.Cu") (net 3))
 (segment (start 47.625 44.515) (end 48.895 44.515) (width 1) (layer "F.Cu") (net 1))
 (segment (start 52.578 40.832) (end 52.578 35.814) (width 1) (layer "F.Cu") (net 1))
 (segment (start 48.895 44.515) (end 52.578 40.832) (width 1) (layer "F.Cu") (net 1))
 (segment (start 31.755 44.196) (end 38.862 44.196) (width 2) (layer "B.Cu") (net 10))
 (segment (start 28.154 47.797) (end 31.755 44.196) (width 2) (layer "B.Cu") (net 10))
 (segment (start 47.244 35.814) (end 47.498 35.814) (width 2) (layer "B.Cu") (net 10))
 (segment (start 38.862 44.196) (end 47.244 35.814) (width 2) (layer "B.Cu") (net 10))
 (segment (start 18.034 52.07) (end 26.162 43.942) (width 0.2) (layer "F.Cu") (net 7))
 (segment (start 26.162 37.589) (end 28.154 35.597) (width 0.2) (layer "F.Cu") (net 7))
 (segment (start 26.162 43.942) (end 26.162 37.589) (width 0.2) (layer "F.Cu") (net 7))
 (segment (start 21.91 41.214) (end 22.86 42.164) (width 0.2) (layer "F.Cu") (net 9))
 (segment (start 21.91 38.9835) (end 21.91 41.214) (width 0.2) (layer "F.Cu") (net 9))
 (via (at 22.86 42.164) (size 0.6) (drill 0.3) (layers "F.Cu" "B.Cu") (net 9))
 (segment (start 22.86 42.164) (end 23.368 42.164) (width 0.2) (layer "B.Cu") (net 9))
 (segment (start 23.368 42.164) (end 24.638 43.434) (width 0.2) (layer "B.Cu") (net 9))
 (segment (start 24.638 50.546) (end 23.114 52.07) (width 0.2) (layer "B.Cu") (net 9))
 (segment (start 24.638 43.434) (end 24.638 50.546) (width 0.2) (layer "B.Cu") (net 9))
 (segment (start 23.81 44.638) (end 23.876 44.704) (width 0.2) (layer "F.Cu") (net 8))
 (segment (start 23.81 38.9835) (end 23.81 44.638) (width 0.2) (layer "F.Cu") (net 8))
 (via (at 23.876 44.704) (size 0.6) (drill 0.3) (layers "F.Cu" "B.Cu") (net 8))
 (segment (start 23.876 48.768) (end 23.876 44.704) (width 0.2) (layer "B.Cu") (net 8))
 (segment (start 20.574 52.07) (end 23.876 48.768) (width 0.2) (layer "B.Cu") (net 8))
 (segment (start 36.053 31.496) (end 40.154 35.597) (width 0.2) (layer "F.Cu") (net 12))
 (segment (start 28.0725 31.496) (end 36.053 31.496) (width 0.2) (layer "F.Cu") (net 12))
 (segment (start 22.86 36.7085) (end 28.0725 31.496) (width 0.2) (layer "F.Cu") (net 12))
 (segment (start 45.085 44.515) (end 46.355 44.515) (width 1) (layer "F.Cu") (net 2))
 (segment (start 34.154 33.597) (end 34.167 33.597) (width 1) (layer "F.Cu") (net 2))
 (segment (start 43.18 42.61) (end 43.18 43.434) (width 2) (layer "F.Cu") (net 2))
 (segment (start 34.167 33.597) (end 43.18 42.61) (width 2) (layer "F.Cu") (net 2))
 (segment (start 45.675 47.797) (end 57.658 35.814) (width 2) (layer "B.Cu") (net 11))
 (segment (start 45.675 47.797) (end 40.154 47.797) (width 2) (layer "B.Cu") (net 11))
 (segment (start 56.896 51.562) (end 55.3935 53.0645) (width 0.2) (layer "F.Cu") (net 6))
 (segment (start 48.895 52.9375) (end 49.022 53.0645) (width 0.2) (layer "F.Cu") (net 6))
 (segment (start 55.3935 53.0645) (end 49.022 53.0645) (width 0.2) (layer "F.Cu") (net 6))
 (segment (start 48.895 49.465) (end 48.895 52.9375) (width 0.2) (layer "F.Cu") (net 6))
 (segment (start 59.436 51.562) (end 57.404 49.53) (width 0.2) (layer "F.Cu") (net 5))
 (segment (start 47.926001 48.189) (end 47.625 48.490001) (width 0.2) (layer "F.Cu") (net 5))
 (segment (start 57.404 49.53) (end 55.372 49.53) (width 0.2) (layer "F.Cu") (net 5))
 (segment (start 47.625 48.490001) (end 47.625 49.465) (width 0.2) (layer "F.Cu") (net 5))
 (segment (start 54.031 48.189) (end 47.926001 48.189) (width 0.2) (layer "F.Cu") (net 5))
 (segment (start 55.372 49.53) (end 54.031 48.189) (width 0.2) (layer "F.Cu") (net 5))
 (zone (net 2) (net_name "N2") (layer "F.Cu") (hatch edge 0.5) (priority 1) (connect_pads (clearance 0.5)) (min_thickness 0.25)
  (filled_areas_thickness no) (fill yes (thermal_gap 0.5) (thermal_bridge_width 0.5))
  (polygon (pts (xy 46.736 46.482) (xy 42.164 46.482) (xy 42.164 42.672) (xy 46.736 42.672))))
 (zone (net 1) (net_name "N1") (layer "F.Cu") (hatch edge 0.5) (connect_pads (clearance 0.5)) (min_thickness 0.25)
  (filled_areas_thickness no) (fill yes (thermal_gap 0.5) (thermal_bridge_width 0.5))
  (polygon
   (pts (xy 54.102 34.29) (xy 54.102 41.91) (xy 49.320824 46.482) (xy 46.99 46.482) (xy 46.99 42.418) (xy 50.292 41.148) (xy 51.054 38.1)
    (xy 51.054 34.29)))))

